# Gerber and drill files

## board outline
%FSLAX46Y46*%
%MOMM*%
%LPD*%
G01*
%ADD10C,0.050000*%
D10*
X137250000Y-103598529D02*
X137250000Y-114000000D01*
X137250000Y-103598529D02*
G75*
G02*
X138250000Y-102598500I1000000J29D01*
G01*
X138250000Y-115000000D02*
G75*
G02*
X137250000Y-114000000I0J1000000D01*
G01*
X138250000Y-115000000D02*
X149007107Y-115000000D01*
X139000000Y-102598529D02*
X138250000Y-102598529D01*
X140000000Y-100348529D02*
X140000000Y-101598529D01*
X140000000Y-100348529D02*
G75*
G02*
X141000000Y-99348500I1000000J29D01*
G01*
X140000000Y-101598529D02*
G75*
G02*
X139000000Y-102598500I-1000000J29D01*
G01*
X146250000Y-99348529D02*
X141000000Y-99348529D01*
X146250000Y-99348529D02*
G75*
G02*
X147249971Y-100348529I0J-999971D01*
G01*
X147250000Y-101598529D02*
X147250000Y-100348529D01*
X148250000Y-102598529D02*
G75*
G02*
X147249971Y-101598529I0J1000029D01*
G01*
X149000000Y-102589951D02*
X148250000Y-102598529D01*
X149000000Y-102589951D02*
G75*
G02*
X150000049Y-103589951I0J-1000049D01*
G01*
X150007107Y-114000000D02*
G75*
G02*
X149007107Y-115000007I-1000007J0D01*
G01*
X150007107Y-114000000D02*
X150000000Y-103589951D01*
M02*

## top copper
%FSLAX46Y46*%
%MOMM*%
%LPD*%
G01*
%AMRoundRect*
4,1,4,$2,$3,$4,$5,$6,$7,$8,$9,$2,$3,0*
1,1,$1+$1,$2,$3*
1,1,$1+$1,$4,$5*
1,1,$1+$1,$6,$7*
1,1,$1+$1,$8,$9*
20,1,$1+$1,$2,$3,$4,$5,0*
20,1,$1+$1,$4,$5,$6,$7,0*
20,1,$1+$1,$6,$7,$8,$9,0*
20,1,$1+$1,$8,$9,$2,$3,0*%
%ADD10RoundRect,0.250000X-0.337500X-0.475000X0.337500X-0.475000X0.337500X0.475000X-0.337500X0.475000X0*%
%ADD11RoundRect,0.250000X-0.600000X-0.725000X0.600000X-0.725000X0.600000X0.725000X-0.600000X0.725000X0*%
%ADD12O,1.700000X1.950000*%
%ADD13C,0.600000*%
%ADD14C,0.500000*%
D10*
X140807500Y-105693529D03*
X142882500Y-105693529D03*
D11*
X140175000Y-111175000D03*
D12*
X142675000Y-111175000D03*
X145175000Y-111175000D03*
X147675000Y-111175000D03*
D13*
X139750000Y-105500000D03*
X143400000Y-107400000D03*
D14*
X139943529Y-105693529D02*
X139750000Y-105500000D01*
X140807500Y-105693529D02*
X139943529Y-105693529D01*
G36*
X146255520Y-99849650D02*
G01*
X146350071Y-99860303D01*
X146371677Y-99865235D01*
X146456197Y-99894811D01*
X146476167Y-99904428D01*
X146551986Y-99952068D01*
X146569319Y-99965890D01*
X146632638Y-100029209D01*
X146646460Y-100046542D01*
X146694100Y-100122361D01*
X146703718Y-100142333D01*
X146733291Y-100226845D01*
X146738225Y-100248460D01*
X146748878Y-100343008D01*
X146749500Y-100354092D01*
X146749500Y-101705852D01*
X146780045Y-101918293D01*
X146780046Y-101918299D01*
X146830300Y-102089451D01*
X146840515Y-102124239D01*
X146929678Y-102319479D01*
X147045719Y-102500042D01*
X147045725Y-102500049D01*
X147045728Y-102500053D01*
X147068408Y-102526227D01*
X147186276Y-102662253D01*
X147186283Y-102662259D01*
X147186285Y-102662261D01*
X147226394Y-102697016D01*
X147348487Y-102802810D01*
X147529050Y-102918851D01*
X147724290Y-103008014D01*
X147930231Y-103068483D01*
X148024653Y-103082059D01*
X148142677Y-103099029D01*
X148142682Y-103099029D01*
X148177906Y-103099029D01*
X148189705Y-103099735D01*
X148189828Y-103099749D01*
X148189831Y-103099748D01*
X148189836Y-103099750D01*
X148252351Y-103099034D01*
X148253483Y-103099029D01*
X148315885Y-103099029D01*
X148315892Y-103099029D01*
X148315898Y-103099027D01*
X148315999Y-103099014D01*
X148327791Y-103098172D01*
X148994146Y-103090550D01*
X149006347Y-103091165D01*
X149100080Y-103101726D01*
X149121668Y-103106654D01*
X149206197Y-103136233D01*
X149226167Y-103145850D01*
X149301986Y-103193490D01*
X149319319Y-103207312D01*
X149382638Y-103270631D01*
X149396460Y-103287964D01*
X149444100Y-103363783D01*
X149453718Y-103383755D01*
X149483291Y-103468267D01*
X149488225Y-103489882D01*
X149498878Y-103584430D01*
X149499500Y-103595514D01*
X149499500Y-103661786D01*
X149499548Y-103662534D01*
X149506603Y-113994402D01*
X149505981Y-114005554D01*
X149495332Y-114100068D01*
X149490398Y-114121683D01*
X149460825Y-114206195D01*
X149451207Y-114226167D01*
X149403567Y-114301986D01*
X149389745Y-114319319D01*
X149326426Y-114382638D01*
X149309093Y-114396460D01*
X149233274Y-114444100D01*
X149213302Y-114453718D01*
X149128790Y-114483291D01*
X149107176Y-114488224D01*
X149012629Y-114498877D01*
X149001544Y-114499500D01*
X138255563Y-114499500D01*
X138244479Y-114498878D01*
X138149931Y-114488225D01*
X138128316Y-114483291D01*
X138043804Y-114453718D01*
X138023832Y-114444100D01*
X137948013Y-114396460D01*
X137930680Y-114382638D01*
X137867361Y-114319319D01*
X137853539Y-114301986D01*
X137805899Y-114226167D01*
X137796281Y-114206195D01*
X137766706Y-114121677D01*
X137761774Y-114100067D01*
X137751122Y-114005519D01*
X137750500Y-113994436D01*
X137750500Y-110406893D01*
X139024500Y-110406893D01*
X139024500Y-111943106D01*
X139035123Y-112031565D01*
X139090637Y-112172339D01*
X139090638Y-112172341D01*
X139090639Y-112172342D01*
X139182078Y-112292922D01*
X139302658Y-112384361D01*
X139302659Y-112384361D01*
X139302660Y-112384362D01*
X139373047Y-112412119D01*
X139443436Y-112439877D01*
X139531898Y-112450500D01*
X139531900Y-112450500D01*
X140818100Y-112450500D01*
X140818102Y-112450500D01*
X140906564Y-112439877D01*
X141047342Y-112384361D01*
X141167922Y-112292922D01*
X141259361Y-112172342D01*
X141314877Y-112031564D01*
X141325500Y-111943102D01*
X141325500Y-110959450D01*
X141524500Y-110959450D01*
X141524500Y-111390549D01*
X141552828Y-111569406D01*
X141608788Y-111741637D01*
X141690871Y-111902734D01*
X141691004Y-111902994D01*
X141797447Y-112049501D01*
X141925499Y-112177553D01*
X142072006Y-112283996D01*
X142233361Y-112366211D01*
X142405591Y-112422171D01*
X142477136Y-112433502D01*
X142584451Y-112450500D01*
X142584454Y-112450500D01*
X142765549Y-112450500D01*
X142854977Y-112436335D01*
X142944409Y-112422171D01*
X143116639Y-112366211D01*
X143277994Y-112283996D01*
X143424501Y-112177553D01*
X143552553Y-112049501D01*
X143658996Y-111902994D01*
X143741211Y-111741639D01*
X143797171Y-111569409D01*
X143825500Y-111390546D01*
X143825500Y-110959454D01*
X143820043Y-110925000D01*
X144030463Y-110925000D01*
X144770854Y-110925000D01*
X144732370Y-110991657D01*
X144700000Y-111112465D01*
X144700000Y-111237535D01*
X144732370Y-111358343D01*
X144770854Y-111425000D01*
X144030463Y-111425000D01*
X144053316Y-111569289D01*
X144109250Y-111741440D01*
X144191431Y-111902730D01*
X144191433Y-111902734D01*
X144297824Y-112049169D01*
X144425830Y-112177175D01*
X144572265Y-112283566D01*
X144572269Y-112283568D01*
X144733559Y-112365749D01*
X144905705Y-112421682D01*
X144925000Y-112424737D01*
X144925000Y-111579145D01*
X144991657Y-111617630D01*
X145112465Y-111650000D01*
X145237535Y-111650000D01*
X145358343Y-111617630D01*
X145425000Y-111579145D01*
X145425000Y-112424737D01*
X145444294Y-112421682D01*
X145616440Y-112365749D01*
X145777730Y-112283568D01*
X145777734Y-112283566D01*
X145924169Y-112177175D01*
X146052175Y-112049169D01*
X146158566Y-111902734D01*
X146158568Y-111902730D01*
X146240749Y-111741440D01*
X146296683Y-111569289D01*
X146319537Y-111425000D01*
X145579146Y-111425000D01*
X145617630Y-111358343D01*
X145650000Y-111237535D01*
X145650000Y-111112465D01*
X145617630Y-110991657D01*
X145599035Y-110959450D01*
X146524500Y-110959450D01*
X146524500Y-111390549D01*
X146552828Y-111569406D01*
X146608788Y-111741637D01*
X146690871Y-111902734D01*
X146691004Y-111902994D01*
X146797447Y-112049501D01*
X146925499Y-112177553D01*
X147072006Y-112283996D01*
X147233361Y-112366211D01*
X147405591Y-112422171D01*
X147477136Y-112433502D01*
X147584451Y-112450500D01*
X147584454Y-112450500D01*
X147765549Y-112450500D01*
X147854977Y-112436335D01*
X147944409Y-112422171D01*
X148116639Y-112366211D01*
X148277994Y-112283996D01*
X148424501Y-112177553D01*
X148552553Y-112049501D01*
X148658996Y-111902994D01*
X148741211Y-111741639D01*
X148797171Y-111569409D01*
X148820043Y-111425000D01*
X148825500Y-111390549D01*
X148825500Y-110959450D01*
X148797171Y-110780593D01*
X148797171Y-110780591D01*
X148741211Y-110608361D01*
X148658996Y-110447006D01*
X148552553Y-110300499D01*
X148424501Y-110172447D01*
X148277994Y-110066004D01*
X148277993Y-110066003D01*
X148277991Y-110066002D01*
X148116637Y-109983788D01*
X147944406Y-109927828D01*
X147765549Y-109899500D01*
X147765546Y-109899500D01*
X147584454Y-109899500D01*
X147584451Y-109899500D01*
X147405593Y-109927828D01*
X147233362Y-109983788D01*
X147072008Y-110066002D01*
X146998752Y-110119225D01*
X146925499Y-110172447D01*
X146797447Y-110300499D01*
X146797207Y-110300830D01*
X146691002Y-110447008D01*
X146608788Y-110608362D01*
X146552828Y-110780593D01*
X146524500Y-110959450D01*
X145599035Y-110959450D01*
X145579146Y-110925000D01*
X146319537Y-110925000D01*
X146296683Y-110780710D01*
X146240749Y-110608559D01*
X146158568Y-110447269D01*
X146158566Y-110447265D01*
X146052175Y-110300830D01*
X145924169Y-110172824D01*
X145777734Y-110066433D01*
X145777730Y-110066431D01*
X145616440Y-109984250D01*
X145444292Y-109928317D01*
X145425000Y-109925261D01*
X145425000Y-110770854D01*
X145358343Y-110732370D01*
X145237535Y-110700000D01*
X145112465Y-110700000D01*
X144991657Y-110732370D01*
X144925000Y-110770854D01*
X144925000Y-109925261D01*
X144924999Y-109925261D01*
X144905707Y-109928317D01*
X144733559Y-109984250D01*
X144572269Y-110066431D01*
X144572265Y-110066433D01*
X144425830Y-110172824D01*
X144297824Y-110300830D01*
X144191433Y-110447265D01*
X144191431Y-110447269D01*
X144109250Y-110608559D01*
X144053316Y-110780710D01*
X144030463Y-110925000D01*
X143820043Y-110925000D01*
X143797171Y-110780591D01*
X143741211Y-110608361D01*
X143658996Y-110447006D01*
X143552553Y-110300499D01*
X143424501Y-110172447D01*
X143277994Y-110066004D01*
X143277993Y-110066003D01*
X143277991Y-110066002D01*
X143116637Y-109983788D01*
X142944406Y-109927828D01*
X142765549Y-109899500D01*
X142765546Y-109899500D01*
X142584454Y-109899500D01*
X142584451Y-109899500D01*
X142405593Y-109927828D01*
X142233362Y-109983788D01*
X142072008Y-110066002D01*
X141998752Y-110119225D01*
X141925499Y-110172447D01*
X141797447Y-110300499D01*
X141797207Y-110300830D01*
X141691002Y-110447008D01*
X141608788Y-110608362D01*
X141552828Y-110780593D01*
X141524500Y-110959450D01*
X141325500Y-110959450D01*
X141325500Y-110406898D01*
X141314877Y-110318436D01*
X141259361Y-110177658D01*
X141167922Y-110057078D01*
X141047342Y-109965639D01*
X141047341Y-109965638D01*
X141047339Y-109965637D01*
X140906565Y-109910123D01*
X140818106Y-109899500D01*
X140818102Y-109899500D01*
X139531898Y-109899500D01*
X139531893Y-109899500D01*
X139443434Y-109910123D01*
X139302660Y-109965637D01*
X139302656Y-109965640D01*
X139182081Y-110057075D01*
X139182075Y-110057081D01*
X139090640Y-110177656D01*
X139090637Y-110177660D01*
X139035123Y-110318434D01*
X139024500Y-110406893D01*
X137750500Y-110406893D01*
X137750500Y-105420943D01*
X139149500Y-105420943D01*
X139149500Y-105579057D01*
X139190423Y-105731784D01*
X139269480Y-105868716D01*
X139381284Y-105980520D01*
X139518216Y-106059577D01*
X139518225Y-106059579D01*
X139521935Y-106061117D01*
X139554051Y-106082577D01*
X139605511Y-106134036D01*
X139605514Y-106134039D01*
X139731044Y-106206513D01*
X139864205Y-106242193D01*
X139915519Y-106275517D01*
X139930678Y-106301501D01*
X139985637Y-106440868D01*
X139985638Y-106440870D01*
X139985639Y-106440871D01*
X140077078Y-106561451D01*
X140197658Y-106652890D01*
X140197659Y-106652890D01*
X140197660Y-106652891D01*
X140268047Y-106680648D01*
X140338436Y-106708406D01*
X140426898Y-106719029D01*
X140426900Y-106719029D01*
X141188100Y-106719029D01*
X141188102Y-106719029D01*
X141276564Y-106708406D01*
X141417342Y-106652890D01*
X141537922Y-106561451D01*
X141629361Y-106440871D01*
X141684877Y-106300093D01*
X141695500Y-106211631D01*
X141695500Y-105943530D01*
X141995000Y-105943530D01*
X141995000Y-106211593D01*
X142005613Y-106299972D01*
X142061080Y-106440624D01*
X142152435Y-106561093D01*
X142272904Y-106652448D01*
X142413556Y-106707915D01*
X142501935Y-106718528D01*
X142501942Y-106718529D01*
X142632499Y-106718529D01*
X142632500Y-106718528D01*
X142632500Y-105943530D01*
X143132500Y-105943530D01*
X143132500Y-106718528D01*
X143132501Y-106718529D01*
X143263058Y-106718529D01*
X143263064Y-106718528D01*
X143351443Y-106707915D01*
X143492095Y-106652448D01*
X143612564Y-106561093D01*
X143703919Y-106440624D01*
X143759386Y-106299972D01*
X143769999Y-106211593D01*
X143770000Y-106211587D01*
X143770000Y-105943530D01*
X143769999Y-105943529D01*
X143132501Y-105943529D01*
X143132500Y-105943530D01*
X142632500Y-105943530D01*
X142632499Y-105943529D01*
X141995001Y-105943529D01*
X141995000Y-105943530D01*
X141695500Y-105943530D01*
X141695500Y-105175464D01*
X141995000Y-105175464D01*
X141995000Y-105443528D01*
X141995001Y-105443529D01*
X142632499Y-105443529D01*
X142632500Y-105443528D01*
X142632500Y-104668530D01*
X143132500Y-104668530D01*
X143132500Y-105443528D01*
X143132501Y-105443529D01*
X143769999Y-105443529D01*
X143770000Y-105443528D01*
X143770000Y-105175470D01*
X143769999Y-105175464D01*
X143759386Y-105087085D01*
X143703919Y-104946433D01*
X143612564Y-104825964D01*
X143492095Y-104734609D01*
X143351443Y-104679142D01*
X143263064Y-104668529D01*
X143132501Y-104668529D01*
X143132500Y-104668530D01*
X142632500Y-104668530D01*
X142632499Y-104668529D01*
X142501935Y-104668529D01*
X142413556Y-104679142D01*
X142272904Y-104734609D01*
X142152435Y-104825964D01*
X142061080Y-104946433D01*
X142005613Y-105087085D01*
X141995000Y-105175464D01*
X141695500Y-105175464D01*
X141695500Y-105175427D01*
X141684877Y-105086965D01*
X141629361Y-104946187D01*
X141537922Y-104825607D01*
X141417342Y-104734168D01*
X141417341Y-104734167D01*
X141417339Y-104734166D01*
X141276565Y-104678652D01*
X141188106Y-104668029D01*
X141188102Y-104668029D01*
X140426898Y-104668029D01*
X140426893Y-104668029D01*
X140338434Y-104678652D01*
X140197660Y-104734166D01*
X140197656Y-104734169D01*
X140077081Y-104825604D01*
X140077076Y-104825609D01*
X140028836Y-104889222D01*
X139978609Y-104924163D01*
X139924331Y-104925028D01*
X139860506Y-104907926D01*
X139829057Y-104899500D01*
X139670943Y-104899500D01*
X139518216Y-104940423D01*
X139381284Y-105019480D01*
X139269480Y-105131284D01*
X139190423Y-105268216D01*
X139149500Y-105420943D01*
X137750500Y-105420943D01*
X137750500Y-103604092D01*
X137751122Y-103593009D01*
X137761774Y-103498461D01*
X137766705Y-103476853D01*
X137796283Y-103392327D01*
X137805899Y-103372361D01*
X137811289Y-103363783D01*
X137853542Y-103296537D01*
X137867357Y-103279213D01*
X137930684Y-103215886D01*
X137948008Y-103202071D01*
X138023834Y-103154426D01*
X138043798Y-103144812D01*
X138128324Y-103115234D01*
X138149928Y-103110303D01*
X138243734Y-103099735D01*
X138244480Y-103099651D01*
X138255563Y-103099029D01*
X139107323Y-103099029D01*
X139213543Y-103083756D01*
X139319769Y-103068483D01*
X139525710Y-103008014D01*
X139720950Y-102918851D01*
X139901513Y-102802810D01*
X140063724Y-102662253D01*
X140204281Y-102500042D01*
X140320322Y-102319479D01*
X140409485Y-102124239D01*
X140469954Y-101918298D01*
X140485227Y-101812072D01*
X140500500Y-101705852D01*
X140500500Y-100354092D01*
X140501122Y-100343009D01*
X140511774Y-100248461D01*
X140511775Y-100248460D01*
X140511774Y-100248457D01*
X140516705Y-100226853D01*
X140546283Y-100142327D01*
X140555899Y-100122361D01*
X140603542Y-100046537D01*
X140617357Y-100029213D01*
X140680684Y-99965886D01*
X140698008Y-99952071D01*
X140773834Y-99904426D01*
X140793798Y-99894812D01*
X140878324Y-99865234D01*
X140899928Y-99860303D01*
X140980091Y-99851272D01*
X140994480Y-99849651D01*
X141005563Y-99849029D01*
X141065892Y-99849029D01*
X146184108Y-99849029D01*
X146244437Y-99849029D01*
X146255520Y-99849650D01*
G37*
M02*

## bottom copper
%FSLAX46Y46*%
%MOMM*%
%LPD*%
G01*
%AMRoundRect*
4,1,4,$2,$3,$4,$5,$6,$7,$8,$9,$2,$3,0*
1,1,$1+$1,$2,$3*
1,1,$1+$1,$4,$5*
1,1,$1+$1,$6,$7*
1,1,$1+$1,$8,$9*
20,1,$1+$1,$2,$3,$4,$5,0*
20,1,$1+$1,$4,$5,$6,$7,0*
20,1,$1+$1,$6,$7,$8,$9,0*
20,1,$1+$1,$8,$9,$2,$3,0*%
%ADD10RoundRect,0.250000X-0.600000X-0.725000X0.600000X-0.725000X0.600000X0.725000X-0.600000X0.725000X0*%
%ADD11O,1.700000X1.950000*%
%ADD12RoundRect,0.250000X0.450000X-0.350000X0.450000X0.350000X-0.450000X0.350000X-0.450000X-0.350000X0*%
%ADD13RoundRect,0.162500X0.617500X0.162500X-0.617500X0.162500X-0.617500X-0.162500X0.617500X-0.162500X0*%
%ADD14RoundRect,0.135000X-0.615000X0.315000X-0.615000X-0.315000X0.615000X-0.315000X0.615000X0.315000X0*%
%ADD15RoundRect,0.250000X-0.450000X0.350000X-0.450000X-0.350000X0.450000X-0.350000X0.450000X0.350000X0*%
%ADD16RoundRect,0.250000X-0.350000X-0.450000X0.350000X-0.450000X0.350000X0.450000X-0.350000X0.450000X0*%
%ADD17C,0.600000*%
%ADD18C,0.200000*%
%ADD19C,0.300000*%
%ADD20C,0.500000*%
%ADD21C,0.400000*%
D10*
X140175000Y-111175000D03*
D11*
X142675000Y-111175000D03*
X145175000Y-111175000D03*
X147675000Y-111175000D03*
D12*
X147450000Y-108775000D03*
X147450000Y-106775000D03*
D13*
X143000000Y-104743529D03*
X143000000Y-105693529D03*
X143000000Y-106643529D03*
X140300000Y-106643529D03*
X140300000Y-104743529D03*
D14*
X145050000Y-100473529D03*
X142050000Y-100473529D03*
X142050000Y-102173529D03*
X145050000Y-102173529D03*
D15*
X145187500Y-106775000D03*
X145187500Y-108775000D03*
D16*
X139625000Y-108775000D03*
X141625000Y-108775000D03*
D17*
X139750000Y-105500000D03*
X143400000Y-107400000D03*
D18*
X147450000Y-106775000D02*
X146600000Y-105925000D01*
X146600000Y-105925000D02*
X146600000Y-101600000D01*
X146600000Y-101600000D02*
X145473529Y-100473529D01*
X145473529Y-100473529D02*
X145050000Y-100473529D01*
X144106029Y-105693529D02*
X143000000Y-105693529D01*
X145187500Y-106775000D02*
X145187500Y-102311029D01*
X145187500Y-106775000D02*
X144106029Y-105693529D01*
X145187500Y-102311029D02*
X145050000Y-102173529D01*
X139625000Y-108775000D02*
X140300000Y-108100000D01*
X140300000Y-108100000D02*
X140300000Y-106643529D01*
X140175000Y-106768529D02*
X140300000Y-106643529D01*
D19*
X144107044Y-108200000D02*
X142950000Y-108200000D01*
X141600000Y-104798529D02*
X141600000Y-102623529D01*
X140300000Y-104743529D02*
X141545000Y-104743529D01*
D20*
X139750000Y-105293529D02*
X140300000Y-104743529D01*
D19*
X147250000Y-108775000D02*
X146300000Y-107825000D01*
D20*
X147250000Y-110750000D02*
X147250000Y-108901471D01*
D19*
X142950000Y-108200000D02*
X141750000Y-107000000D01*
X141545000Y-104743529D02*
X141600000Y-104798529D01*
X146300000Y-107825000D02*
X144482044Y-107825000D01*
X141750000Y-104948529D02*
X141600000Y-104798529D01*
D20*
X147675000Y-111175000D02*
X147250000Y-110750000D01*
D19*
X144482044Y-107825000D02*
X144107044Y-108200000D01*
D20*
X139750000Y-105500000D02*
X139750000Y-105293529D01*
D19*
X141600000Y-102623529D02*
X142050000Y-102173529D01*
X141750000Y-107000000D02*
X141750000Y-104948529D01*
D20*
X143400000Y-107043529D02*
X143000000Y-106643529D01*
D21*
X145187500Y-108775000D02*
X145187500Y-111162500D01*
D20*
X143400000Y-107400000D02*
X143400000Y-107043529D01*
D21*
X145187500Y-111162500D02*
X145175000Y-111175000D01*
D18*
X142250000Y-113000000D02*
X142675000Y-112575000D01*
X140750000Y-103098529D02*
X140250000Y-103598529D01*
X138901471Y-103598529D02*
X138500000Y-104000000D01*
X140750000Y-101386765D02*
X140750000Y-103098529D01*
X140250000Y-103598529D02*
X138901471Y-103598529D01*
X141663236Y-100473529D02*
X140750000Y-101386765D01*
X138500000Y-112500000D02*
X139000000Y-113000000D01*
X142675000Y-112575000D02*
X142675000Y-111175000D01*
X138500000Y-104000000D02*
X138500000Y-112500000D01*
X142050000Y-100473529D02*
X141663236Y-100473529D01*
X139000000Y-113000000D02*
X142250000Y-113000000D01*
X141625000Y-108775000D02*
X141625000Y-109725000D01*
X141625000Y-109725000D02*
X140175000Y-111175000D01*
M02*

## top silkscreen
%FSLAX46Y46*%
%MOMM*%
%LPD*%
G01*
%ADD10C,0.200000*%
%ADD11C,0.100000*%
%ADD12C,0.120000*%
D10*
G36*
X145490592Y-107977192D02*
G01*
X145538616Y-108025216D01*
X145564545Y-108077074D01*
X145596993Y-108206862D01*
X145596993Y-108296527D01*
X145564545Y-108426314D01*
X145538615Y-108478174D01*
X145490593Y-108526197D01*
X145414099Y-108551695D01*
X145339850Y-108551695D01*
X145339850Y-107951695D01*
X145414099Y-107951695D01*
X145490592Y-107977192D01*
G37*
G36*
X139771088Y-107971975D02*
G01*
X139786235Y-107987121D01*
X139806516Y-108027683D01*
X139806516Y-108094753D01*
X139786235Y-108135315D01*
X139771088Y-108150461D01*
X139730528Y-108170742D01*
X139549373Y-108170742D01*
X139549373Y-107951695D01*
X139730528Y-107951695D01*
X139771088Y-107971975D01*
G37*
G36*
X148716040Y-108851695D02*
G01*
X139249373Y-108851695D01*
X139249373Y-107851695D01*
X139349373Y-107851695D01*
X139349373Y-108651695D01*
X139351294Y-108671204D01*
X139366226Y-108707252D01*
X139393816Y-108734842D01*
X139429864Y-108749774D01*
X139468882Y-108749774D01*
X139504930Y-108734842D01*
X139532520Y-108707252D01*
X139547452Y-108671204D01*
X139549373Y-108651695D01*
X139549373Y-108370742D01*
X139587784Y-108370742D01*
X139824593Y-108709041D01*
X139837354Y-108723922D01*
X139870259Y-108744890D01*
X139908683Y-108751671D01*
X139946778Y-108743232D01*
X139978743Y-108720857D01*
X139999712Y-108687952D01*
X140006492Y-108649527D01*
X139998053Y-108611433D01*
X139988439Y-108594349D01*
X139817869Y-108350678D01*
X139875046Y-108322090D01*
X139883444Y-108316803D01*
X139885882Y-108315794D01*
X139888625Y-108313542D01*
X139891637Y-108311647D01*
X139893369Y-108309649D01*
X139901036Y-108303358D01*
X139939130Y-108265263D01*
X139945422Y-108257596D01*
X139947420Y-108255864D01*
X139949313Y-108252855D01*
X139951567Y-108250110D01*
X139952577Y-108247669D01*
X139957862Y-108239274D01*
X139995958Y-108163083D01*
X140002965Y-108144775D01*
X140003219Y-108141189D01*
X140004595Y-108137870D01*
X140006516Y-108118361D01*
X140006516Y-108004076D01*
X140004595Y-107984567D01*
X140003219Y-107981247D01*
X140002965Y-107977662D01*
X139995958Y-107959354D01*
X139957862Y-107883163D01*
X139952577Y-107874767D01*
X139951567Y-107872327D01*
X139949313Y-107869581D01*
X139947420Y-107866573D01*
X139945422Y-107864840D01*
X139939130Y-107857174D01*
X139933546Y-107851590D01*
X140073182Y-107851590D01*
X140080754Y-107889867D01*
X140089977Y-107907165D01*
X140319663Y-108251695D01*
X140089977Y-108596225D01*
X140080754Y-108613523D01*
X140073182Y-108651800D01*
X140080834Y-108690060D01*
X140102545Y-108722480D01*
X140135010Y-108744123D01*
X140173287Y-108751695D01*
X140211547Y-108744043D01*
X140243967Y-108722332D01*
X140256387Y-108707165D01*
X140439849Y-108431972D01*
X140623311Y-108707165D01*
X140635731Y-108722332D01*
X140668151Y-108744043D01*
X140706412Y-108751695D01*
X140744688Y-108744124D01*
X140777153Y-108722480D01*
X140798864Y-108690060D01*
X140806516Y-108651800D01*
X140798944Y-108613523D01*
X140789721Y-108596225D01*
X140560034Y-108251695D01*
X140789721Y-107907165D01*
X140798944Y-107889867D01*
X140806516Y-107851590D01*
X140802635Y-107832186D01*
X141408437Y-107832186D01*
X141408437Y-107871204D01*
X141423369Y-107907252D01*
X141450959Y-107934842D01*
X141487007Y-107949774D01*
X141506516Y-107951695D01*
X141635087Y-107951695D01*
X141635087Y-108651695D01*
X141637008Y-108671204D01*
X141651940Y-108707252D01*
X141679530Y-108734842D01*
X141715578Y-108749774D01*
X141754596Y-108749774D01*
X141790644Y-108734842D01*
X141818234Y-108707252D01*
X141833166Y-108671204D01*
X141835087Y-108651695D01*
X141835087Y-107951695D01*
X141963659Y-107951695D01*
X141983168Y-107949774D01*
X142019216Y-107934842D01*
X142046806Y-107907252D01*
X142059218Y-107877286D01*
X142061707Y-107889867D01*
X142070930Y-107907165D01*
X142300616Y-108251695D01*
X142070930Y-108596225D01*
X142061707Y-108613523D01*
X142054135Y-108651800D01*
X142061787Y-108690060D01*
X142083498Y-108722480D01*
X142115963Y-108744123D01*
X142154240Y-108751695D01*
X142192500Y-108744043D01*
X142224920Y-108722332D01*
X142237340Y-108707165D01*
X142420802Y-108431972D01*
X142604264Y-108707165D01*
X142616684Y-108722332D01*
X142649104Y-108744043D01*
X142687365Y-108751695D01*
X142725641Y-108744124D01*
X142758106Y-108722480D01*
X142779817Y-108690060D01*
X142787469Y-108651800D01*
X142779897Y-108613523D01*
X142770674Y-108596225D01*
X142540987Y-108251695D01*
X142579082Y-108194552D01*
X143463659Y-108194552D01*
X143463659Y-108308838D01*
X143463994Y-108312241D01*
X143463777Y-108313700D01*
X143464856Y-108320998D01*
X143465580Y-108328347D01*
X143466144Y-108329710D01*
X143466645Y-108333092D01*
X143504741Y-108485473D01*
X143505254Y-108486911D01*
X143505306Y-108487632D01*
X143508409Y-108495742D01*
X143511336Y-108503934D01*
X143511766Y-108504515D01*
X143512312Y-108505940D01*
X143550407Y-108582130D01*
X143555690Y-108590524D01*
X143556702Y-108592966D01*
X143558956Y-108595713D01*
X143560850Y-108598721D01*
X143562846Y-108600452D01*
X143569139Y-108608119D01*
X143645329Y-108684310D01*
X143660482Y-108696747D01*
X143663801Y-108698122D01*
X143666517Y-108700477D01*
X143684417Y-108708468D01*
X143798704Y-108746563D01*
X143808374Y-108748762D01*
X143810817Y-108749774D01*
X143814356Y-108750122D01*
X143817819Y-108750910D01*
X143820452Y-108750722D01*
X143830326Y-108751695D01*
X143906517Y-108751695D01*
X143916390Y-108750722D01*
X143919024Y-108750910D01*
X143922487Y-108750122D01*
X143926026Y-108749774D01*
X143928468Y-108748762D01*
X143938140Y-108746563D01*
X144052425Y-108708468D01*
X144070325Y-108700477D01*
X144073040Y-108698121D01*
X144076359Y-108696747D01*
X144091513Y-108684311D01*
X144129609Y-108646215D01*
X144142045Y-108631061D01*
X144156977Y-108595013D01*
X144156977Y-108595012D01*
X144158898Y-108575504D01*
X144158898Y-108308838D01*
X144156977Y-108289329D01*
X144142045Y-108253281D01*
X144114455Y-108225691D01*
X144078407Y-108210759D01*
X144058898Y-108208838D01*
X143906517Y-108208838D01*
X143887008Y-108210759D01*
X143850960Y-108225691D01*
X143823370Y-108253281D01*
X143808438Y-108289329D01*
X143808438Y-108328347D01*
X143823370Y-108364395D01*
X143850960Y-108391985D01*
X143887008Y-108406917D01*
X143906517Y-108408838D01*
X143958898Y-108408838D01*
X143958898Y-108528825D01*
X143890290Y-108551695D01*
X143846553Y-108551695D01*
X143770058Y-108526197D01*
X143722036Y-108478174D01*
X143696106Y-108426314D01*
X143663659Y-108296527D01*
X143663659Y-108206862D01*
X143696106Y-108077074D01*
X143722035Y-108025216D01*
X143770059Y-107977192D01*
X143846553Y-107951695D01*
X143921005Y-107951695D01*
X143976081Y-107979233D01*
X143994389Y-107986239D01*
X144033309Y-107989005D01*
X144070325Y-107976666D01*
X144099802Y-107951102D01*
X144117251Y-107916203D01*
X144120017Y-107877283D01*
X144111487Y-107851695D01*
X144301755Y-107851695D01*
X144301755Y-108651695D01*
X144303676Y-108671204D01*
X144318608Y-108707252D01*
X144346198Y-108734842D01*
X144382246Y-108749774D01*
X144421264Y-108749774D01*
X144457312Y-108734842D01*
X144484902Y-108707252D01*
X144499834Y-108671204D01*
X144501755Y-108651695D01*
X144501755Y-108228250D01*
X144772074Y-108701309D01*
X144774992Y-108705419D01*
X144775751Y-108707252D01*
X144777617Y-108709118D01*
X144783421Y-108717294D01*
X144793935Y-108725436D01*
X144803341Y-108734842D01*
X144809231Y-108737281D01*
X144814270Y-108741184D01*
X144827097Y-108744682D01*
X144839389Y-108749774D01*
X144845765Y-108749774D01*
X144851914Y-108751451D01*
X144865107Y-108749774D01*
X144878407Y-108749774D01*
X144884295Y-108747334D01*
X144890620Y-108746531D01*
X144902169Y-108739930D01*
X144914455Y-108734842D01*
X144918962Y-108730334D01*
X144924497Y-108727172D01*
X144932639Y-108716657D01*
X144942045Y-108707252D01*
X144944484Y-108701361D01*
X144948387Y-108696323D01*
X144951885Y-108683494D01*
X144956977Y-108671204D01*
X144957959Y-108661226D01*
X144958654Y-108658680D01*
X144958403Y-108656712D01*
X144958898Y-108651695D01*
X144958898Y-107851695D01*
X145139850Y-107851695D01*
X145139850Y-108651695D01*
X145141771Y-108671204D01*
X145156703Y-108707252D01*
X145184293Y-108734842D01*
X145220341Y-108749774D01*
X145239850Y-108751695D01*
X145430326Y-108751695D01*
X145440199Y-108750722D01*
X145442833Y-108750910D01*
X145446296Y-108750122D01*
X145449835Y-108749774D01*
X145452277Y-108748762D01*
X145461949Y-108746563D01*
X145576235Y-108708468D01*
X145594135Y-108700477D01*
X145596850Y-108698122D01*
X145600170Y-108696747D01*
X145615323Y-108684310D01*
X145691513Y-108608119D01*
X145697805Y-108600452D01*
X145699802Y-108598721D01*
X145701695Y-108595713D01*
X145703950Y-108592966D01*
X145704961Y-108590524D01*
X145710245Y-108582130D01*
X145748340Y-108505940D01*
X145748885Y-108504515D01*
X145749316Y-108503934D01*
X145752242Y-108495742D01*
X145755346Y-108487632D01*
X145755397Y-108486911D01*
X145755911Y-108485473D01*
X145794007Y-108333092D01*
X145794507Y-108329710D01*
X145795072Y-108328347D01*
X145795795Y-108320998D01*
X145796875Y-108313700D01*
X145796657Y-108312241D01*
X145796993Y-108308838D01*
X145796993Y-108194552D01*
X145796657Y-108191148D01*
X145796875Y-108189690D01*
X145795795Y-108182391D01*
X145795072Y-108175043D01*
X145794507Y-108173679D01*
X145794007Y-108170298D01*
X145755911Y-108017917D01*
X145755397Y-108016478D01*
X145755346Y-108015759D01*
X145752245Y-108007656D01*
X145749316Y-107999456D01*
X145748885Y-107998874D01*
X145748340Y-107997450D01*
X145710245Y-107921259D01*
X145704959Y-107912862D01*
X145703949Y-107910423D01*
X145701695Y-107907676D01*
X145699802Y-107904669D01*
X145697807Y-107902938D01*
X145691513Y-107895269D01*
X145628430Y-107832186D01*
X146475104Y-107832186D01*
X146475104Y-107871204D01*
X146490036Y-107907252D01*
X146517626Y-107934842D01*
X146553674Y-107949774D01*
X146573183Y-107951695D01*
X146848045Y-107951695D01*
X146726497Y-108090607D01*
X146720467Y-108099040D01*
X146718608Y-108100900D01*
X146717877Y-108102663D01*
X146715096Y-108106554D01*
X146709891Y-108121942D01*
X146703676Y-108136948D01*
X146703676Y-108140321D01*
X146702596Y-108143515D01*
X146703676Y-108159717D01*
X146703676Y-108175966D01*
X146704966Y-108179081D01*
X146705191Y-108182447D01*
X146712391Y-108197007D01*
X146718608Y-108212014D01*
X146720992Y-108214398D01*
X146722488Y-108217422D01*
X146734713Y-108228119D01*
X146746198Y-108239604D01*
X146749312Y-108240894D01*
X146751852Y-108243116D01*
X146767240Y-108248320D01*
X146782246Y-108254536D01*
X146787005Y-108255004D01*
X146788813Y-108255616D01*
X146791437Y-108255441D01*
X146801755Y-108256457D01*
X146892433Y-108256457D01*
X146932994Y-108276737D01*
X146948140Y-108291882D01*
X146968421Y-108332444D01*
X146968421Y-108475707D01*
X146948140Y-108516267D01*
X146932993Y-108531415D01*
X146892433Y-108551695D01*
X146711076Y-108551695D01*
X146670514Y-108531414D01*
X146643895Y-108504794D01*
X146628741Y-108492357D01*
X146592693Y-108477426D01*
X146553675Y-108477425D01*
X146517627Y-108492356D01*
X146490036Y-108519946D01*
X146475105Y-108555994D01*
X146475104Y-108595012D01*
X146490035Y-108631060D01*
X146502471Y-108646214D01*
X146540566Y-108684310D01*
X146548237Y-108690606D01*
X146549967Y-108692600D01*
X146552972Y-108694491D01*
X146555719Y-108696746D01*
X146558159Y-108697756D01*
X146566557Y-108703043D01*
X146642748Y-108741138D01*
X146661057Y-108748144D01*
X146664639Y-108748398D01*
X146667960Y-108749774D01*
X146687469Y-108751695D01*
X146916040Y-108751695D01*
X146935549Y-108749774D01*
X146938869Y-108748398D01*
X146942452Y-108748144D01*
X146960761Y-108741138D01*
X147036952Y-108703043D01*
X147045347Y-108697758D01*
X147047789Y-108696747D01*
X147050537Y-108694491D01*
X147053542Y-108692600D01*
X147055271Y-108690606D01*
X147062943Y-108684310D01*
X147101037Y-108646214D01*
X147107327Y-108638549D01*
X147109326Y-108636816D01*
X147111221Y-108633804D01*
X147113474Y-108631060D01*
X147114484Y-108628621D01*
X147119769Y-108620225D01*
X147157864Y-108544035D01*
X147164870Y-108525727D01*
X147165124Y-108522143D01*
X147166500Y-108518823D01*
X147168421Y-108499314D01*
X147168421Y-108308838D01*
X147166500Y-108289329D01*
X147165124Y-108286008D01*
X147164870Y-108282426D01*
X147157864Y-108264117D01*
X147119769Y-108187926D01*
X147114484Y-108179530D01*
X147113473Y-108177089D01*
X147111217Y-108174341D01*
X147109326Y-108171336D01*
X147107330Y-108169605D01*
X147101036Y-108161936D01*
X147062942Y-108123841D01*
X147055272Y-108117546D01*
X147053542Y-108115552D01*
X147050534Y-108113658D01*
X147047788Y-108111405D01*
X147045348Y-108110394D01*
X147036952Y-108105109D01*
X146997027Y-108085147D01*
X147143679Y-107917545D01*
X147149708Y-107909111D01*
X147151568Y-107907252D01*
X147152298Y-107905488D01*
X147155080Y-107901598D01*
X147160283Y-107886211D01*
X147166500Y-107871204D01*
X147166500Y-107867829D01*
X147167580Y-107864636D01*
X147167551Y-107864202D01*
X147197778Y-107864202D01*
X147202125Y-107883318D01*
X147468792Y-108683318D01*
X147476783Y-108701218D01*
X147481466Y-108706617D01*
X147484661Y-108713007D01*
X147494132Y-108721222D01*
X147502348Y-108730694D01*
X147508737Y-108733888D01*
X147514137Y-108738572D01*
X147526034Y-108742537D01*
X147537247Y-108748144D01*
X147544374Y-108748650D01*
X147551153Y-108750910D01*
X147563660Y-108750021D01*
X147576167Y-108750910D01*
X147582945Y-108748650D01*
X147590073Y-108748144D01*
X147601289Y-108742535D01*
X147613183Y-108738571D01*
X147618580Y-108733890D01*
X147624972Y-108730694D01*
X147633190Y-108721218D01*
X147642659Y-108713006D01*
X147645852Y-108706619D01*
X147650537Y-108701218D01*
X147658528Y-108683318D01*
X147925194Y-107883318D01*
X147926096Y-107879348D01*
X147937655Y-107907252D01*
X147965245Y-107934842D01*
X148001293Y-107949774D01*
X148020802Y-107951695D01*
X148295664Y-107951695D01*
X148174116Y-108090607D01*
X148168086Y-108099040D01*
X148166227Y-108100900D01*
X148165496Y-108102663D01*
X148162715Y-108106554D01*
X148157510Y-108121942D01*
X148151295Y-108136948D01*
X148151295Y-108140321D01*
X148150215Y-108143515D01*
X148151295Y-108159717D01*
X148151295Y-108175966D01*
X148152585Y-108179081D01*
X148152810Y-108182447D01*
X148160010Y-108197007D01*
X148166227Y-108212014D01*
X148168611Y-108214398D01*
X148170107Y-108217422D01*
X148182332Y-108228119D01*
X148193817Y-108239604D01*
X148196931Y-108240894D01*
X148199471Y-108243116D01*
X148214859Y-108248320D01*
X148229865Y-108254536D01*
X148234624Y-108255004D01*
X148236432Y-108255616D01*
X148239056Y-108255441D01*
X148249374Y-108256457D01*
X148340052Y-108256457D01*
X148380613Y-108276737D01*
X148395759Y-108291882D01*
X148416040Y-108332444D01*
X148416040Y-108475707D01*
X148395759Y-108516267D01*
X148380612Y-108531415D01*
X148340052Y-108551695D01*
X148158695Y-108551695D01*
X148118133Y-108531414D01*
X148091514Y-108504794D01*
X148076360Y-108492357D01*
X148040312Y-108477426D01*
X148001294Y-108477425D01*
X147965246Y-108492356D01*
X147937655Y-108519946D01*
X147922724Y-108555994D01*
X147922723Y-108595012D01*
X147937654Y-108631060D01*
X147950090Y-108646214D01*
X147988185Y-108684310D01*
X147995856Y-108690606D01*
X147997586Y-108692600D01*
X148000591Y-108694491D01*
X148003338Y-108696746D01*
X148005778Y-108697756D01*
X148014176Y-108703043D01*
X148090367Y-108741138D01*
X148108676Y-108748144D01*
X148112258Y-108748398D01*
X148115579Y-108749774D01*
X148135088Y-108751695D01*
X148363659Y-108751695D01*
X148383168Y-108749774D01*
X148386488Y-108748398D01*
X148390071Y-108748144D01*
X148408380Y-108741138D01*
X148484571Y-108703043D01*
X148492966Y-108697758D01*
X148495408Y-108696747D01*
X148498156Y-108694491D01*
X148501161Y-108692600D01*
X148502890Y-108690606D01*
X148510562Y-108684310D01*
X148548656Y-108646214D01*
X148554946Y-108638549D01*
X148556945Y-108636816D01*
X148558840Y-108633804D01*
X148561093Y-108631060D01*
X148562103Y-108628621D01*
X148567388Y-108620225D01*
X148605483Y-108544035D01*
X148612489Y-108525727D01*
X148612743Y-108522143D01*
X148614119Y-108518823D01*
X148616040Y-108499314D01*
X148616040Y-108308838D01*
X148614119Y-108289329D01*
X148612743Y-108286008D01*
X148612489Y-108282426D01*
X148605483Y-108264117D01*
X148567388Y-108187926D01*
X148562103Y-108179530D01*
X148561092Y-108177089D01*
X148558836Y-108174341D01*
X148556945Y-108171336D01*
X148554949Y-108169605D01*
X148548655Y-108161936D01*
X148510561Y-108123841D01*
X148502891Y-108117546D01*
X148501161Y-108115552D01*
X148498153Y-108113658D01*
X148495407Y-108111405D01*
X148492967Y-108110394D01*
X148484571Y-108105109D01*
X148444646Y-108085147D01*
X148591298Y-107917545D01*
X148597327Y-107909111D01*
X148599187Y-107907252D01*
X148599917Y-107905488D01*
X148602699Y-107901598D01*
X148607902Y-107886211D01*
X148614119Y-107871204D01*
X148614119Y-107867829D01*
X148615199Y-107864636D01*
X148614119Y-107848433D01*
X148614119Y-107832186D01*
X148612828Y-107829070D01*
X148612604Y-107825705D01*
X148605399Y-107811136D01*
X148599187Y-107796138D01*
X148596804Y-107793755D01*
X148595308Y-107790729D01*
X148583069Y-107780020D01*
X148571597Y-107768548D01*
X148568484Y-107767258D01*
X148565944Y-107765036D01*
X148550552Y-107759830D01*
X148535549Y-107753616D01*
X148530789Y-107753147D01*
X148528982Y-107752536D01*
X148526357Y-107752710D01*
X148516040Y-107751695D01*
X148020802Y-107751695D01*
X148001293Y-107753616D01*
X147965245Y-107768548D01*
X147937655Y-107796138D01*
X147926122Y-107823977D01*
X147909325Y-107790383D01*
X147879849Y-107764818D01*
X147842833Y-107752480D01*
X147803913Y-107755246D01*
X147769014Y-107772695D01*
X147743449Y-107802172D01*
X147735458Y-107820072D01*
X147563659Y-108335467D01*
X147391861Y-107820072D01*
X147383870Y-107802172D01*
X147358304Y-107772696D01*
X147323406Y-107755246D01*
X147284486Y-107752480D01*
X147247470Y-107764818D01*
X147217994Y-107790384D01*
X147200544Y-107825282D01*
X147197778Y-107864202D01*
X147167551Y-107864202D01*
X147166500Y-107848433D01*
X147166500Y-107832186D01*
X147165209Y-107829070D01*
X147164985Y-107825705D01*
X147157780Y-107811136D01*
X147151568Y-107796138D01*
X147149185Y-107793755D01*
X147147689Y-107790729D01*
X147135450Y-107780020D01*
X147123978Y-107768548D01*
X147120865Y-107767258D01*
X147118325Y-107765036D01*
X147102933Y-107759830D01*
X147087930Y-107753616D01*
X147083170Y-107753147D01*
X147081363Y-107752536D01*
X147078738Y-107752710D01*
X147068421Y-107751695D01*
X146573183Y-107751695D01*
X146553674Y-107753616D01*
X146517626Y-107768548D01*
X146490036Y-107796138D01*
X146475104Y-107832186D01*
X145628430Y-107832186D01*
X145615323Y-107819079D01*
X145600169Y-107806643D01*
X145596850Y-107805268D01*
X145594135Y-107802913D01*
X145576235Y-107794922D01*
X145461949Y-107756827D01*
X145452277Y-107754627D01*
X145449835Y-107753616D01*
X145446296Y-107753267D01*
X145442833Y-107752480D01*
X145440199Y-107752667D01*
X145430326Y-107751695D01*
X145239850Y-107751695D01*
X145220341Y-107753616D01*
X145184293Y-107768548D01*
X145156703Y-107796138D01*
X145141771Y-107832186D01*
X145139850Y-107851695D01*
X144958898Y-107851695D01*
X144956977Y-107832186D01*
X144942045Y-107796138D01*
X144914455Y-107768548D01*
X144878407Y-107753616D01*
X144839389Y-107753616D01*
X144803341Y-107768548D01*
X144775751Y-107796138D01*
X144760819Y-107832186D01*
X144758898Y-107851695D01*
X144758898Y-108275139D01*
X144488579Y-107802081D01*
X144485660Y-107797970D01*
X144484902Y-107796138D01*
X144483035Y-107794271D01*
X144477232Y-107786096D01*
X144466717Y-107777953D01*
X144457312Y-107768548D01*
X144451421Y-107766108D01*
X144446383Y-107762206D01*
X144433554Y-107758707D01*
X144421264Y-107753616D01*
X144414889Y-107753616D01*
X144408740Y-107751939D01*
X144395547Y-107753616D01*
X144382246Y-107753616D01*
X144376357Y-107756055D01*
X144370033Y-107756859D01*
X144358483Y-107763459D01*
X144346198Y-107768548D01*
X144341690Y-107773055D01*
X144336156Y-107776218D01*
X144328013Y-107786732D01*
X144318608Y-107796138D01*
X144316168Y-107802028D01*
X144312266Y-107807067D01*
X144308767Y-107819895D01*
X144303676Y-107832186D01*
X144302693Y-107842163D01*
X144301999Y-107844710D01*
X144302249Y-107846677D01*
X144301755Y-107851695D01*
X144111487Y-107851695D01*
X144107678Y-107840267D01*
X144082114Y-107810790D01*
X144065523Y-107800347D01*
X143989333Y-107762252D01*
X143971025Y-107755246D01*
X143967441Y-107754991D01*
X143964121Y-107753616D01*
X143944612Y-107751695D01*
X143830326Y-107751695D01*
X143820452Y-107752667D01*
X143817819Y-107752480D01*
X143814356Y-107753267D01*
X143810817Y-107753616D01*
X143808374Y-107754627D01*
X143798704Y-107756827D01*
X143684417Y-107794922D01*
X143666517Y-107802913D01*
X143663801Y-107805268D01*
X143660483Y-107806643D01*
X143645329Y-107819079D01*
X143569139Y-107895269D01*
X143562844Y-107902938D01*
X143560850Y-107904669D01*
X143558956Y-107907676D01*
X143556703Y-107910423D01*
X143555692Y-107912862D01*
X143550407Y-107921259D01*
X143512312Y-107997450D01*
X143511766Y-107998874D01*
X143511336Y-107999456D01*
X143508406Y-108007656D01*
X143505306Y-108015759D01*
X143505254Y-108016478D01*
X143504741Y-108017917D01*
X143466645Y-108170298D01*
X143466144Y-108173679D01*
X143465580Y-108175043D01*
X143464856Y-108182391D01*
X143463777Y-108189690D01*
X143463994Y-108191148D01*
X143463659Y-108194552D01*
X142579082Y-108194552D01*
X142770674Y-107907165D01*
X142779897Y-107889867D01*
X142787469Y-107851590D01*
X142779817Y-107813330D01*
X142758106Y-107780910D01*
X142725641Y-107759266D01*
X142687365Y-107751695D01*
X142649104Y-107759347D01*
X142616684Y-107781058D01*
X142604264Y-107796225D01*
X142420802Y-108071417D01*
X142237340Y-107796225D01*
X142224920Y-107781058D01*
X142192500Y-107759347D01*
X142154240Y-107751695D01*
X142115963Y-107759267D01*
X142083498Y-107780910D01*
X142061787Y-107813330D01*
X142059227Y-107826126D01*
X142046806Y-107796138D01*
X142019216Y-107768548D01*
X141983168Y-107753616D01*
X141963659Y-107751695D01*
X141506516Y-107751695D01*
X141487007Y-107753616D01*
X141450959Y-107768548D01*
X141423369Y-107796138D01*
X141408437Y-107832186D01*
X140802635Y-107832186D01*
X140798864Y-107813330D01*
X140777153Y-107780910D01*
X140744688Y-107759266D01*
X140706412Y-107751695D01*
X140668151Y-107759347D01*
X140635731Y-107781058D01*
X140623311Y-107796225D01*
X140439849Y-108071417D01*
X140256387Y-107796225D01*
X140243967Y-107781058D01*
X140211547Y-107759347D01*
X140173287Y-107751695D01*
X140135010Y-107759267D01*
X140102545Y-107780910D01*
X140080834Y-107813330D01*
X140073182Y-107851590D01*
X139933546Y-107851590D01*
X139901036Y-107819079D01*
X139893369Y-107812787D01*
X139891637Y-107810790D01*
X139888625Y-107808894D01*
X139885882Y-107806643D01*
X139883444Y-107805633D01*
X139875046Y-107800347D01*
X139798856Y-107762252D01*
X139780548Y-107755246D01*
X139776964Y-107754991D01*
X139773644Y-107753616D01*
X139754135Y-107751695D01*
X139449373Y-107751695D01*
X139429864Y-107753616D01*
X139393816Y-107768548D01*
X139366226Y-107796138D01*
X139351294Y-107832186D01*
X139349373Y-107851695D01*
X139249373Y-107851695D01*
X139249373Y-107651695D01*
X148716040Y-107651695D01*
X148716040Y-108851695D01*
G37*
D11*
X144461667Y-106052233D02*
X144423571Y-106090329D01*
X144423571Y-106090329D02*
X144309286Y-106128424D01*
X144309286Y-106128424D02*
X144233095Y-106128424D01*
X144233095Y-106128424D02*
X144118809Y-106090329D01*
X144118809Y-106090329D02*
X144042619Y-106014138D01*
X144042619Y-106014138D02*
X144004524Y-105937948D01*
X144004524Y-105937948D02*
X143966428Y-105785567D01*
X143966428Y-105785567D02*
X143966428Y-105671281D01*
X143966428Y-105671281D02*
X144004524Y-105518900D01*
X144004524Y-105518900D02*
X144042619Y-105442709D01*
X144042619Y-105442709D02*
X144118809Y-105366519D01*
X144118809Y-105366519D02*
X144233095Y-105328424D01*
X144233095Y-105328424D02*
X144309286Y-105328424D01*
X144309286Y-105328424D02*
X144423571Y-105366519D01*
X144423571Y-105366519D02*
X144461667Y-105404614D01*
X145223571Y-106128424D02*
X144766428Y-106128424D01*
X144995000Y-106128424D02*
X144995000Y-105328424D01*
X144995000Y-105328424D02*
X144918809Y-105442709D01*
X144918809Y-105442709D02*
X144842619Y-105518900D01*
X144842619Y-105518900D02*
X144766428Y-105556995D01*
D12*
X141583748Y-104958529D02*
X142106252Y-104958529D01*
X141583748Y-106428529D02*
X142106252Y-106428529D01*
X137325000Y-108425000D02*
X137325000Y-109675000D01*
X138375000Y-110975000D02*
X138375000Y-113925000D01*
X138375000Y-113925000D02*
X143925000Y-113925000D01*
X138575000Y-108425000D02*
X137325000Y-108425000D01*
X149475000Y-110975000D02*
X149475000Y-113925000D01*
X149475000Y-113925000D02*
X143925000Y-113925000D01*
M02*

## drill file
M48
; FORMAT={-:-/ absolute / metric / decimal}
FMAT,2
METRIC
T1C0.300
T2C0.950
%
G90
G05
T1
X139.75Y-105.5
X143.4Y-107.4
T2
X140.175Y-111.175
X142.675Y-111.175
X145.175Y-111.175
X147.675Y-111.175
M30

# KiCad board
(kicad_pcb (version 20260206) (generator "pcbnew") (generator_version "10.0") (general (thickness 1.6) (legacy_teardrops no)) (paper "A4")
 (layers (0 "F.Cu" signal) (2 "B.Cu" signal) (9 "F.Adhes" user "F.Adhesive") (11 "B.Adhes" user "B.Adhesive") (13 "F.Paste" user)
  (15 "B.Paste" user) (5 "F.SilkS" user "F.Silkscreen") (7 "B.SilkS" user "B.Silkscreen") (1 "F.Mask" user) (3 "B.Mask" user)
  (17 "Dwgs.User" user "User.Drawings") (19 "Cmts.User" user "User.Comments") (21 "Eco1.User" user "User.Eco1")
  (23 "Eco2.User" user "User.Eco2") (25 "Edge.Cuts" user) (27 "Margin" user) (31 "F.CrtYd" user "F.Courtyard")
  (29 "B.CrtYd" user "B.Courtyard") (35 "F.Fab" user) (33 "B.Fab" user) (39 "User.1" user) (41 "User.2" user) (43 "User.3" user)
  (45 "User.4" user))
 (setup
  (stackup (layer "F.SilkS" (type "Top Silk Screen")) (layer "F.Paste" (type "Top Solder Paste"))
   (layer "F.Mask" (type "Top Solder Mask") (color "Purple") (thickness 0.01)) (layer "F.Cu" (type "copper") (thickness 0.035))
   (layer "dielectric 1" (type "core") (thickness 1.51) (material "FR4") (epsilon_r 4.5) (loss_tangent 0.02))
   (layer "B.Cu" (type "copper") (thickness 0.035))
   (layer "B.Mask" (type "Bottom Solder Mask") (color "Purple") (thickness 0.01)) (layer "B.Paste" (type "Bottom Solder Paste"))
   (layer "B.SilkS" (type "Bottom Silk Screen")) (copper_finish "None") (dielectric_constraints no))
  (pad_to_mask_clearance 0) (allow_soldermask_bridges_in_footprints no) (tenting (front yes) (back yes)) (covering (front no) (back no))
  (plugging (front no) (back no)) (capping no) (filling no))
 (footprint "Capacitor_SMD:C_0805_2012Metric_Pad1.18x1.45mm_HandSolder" (layer "F.Cu") (at 141.845 105.693529)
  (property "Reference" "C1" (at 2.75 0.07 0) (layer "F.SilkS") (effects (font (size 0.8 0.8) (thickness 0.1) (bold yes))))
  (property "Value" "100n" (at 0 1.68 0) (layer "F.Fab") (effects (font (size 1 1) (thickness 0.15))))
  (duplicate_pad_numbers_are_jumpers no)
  (fp_line (start -0.261252 -0.735) (end 0.261252 -0.735) (stroke (width 0.12) (type solid)) (layer "F.SilkS"))
  (fp_line (start -0.261252 0.735) (end 0.261252 0.735) (stroke (width 0.12) (type solid)) (layer "F.SilkS"))
  (pad "1" smd roundrect (at -1.0375 0) (size 1.175 1.45) (layers "F.Cu" "F.Mask" "F.Paste") (roundrect_rratio 0.212766) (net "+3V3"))
  (pad "2" smd roundrect (at 1.0375 0) (size 1.175 1.45) (layers "F.Cu" "F.Mask" "F.Paste") (roundrect_rratio 0.212766) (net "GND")))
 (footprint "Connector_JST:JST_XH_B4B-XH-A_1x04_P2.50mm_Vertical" (layer "F.Cu") (at 140.175 111.175)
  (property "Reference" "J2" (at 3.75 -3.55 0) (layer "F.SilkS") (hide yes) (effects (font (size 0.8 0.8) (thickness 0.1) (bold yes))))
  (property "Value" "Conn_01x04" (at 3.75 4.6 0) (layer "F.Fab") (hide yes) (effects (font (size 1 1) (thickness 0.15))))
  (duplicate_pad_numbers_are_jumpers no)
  (fp_line (start -2.85 -2.75) (end -2.85 -1.5) (stroke (width 0.12) (type solid)) (layer "F.SilkS"))
  (fp_line (start -1.8 -0.2) (end -1.8 2.75) (stroke (width 0.12) (type solid)) (layer "F.SilkS"))
  (fp_line (start -1.8 2.75) (end 3.75 2.75) (stroke (width 0.12) (type solid)) (layer "F.SilkS"))
  (fp_line (start -1.6 -2.75) (end -2.85 -2.75) (stroke (width 0.12) (type solid)) (layer "F.SilkS"))
  (fp_line (start 9.3 -0.2) (end 9.3 2.75) (stroke (width 0.12) (type solid)) (layer "F.SilkS"))
  (fp_line (start 9.3 2.75) (end 3.75 2.75) (stroke (width 0.12) (type solid)) (layer "F.SilkS"))
  (pad "1" thru_hole roundrect (at 0 0) (size 1.7 1.95) (drill 0.95) (layers "*.Cu" "*.Mask") (remove_unused_layers no)
   (roundrect_rratio 0.147059) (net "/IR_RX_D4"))
  (pad "2" thru_hole oval (at 2.5 0) (size 1.7 1.95) (drill 0.95) (layers "*.Cu" "*.Mask") (remove_unused_layers no) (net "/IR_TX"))
  (pad "3" thru_hole oval (at 5 0) (size 1.7 1.95) (drill 0.95) (layers "*.Cu" "*.Mask") (remove_unused_layers no) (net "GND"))
  (pad "4" thru_hole oval (at 7.5 0) (size 1.7 1.95) (drill 0.95) (layers "*.Cu" "*.Mask") (remove_unused_layers no) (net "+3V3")))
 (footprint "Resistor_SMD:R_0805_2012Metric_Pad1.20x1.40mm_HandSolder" (layer "B.Cu") (at 147.45 107.775 90)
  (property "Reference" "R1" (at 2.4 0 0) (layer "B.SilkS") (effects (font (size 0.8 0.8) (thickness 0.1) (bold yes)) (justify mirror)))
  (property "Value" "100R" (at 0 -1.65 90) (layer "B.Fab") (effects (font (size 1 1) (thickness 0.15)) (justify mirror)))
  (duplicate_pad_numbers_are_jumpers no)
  (pad "1" smd roundrect (at -1 0 90) (size 1.2 1.4) (layers "B.Cu" "B.Mask" "B.Paste") (roundrect_rratio 0.208333) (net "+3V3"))
  (pad "2" smd roundrect (at 1 0 90) (size 1.2 1.4) (layers "B.Cu" "B.Mask" "B.Paste") (roundrect_rratio 0.208333) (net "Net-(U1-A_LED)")))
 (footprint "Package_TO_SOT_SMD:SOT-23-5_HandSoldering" (layer "B.Cu") (at 141.65 105.693529 180)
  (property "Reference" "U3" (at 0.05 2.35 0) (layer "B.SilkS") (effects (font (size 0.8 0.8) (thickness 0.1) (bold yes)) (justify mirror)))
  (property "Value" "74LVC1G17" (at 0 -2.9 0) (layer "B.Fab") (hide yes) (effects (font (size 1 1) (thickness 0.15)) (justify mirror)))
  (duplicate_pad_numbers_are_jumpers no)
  (pad "1" smd roundrect (at -1.35 0.95 180) (size 1.56 0.65) (layers "B.Cu" "B.Mask" "B.Paste") (roundrect_rratio 0.25)
   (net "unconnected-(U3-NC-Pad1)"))
  (pad "2" smd roundrect (at -1.35 0 180) (size 1.56 0.65) (layers "B.Cu" "B.Mask" "B.Paste") (roundrect_rratio 0.25) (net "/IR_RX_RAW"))
  (pad "3" smd roundrect (at -1.35 -0.95 180) (size 1.56 0.65) (layers "B.Cu" "B.Mask" "B.Paste") (roundrect_rratio 0.25) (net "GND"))
  (pad "4" smd roundrect (at 1.35 -0.95 180) (size 1.56 0.65) (layers "B.Cu" "B.Mask" "B.Paste") (roundrect_rratio 0.25)
   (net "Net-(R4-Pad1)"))
  (pad "5" smd roundrect (at 1.35 0.95 180) (size 1.56 0.65) (layers "B.Cu" "B.Mask" "B.Paste") (roundrect_rratio 0.25) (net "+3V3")))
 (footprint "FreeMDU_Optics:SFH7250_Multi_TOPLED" (layer "B.Cu") (at 143.55 101.323529 -90)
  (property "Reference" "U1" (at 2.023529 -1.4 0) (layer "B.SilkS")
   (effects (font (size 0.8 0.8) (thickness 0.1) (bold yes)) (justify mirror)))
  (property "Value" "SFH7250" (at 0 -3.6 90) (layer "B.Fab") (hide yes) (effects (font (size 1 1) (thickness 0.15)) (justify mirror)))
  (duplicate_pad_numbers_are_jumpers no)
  (pad "1" smd roundrect (at -0.85 -1.5 270) (size 0.9 1.5) (layers "B.Cu" "B.Mask" "B.Paste") (roundrect_rratio 0.15)
   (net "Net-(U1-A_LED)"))
  (pad "2" smd roundrect (at -0.85 1.5 270) (size 0.9 1.5) (layers "B.Cu" "B.Mask" "B.Paste") (roundrect_rratio 0.15) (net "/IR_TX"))
  (pad "3" smd roundrect (at 0.85 1.5 270) (size 0.9 1.5) (layers "B.Cu" "B.Mask" "B.Paste") (roundrect_rratio 0.15) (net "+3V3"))
  (pad "4" smd roundrect (at 0.85 -1.5 270) (size 0.9 1.5) (layers "B.Cu" "B.Mask" "B.Paste") (roundrect_rratio 0.15) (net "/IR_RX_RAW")))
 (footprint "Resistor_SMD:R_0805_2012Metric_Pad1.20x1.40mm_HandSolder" (layer "B.Cu") (at 145.1875 107.775 -90)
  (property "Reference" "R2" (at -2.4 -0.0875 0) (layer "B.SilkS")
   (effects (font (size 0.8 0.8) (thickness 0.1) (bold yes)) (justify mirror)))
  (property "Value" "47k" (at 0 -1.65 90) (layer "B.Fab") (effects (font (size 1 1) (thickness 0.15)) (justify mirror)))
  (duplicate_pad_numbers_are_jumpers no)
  (pad "1" smd roundrect (at -1 0 270) (size 1.2 1.4) (layers "B.Cu" "B.Mask" "B.Paste") (roundrect_rratio 0.208333) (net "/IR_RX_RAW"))
  (pad "2" smd roundrect (at 1 0 270) (size 1.2 1.4) (layers "B.Cu" "B.Mask" "B.Paste") (roundrect_rratio 0.208333) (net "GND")))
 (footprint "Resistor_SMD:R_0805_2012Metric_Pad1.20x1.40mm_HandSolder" (layer "B.Cu") (at 140.625 108.775)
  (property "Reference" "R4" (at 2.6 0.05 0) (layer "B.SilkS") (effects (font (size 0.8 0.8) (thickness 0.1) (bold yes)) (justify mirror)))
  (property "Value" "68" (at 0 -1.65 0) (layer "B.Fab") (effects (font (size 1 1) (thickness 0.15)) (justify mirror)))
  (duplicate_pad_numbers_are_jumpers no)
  (pad "1" smd roundrect (at -1 0) (size 1.2 1.4) (layers "B.Cu" "B.Mask" "B.Paste") (roundrect_rratio 0.208333) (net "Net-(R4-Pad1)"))
  (pad "2" smd roundrect (at 1 0) (size 1.2 1.4) (layers "B.Cu" "B.Mask" "B.Paste") (roundrect_rratio 0.208333) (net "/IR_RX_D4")))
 (gr_line (start 137.25 103.598529) (end 137.25 114) (stroke (width 0.05) (type default)) (layer "Edge.Cuts"))
 (gr_arc (start 137.25 103.598529) (mid 137.542893 102.891422) (end 138.25 102.598529) (stroke (width 0.05) (type default))
  (layer "Edge.Cuts"))
 (gr_arc (start 138.25 115) (mid 137.542893 114.707107) (end 137.25 114) (stroke (width 0.05) (type default)) (layer "Edge.Cuts"))
 (gr_line (start 138.25 115) (end 149.007107 115) (stroke (width 0.05) (type default)) (layer "Edge.Cuts"))
 (gr_line (start 139 102.598529) (end 138.25 102.598529) (stroke (width 0.05) (type default)) (layer "Edge.Cuts"))
 (gr_line (start 140 100.348529) (end 140 101.598529) (stroke (width 0.05) (type default)) (layer "Edge.Cuts"))
 (gr_arc (start 140 100.348529) (mid 140.292893 99.641422) (end 141 99.348529) (stroke (width 0.05) (type default)) (layer "Edge.Cuts"))
 (gr_arc (start 140 101.598529) (mid 139.707107 102.305636) (end 139 102.598529) (stroke (width 0.05) (type default)) (layer "Edge.Cuts"))
 (gr_line (start 146.25 99.348529) (end 141 99.348529) (stroke (width 0.05) (type default)) (layer "Edge.Cuts"))
 (gr_arc (start 146.25 99.348529) (mid 146.957107 99.641422) (end 147.25 100.348529) (stroke (width 0.05) (type default))
  (layer "Edge.Cuts"))
 (gr_line (start 147.25 101.598529) (end 147.25 100.348529) (stroke (width 0.05) (type default)) (layer "Edge.Cuts"))
 (gr_arc (start 148.25 102.598529) (mid 147.542893 102.305636) (end 147.25 101.598529) (stroke (width 0.05) (type default))
  (layer "Edge.Cuts"))
 (gr_line (start 149 102.589951) (end 148.25 102.598529) (stroke (width 0.05) (type default)) (layer "Edge.Cuts"))
 (gr_arc (start 149 102.589951) (mid 149.707107 102.882844) (end 150 103.589951) (stroke (width 0.05) (type default)) (layer "Edge.Cuts"))
 (gr_arc (start 150.007107 114) (mid 149.714214 114.707107) (end 149.007107 115) (stroke (width 0.05) (type default)) (layer "Edge.Cuts"))
 (gr_line (start 150.007107 114) (end 150 103.589951) (stroke (width 0.05) (type default)) (layer "Edge.Cuts"))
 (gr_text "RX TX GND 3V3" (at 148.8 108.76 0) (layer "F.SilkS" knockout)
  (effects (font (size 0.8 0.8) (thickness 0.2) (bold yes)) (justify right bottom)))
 (segment (start 147.45 106.775) (end 146.6 105.925) (width 0.2) (layer "B.Cu") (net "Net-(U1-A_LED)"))
 (segment (start 146.6 105.925) (end 146.6 101.6) (width 0.2) (layer "B.Cu") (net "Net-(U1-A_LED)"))
 (segment (start 146.6 101.6) (end 145.473529 100.473529) (width 0.2) (layer "B.Cu") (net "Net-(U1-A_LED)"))
 (segment (start 145.473529 100.473529) (end 145.05 100.473529) (width 0.2) (layer "B.Cu") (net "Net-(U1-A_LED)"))
 (segment (start 144.106029 105.693529) (end 143 105.693529) (width 0.2) (layer "B.Cu") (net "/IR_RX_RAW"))
 (segment (start 145.1875 106.775) (end 145.1875 102.311029) (width 0.2) (layer "B.Cu") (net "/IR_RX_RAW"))
 (segment (start 145.1875 106.775) (end 144.106029 105.693529) (width 0.2) (layer "B.Cu") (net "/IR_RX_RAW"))
 (segment (start 145.1875 102.311029) (end 145.05 102.173529) (width 0.2) (layer "B.Cu") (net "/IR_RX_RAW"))
 (segment (start 139.625 108.775) (end 140.3 108.1) (width 0.2) (layer "B.Cu") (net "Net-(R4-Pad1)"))
 (segment (start 140.3 108.1) (end 140.3 106.643529) (width 0.2) (layer "B.Cu") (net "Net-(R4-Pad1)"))
 (segment (start 140.175 106.768529) (end 140.3 106.643529) (width 0.2) (layer "B.Cu") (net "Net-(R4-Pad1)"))
 (segment (start 139.943529 105.693529) (end 139.75 105.5) (width 0.5) (layer "F.Cu") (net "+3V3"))
 (segment (start 140.8075 105.693529) (end 139.943529 105.693529) (width 0.5) (layer "F.Cu") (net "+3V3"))
 (via (at 139.75 105.5) (size 0.6) (drill 0.3) (layers "F.Cu" "B.Cu") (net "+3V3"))
 (segment (start 144.107044 108.2) (end 142.95 108.2) (width 0.3) (layer "B.Cu") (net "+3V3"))
 (segment (start 141.6 104.798529) (end 141.6 102.623529) (width 0.3) (layer "B.Cu") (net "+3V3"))
 (segment (start 140.3 104.743529) (end 141.545 104.743529) (width 0.3) (layer "B.Cu") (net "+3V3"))
 (segment (start 139.75 105.293529) (end 140.3 104.743529) (width 0.5) (layer "B.Cu") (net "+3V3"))
 (segment (start 147.25 108.775) (end 146.3 107.825) (width 0.3) (layer "B.Cu") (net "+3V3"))
 (segment (start 147.25 110.75) (end 147.25 108.901471) (width 0.5) (layer "B.Cu") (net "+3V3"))
 (segment (start 142.95 108.2) (end 141.75 107) (width 0.3) (layer "B.Cu") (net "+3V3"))
 (segment (start 141.545 104.743529) (end 141.6 104.798529) (width 0.3) (layer "B.Cu") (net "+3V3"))
 (segment (start 146.3 107.825) (end 144.482044 107.825) (width 0.3) (layer "B.Cu") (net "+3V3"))
 (segment (start 141.75 104.948529) (end 141.6 104.798529) (width 0.3) (layer "B.Cu") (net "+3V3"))
 (segment (start 147.675 111.175) (end 147.25 110.75) (width 0.5) (layer "B.Cu") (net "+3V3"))
 (segment (start 144.482044 107.825) (end 144.107044 108.2) (width 0.3) (layer "B.Cu") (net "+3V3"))
 (segment (start 139.75 105.5) (end 139.75 105.293529) (width 0.5) (layer "B.Cu") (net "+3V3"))
 (segment (start 141.6 102.623529) (end 142.05 102.173529) (width 0.3) (layer "B.Cu") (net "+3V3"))
 (segment (start 141.75 107) (end 141.75 104.948529) (width 0.3) (layer "B.Cu") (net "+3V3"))
 (via (at 143.4 107.4) (size 0.6) (drill 0.3) (layers "F.Cu" "B.Cu") (free yes) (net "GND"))
 (segment (start 143.4 107.043529) (end 143 106.643529) (width 0.5) (layer "B.Cu") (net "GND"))
 (segment (start 145.1875 108.775) (end 145.1875 111.1625) (width 0.4) (layer "B.Cu") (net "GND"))
 (segment (start 143.4 107.4) (end 143.4 107.043529) (width 0.5) (layer "B.Cu") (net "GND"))
 (segment (start 145.1875 111.1625) (end 145.175 111.175) (width 0.4) (layer "B.Cu") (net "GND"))
 (segment (start 142.25 113) (end 142.675 112.575) (width 0.2) (layer "B.Cu") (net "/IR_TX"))
 (segment (start 140.75 103.098529) (end 140.25 103.598529) (width 0.2) (layer "B.Cu") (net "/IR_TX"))
 (segment (start 138.901471 103.598529) (end 138.5 104) (width 0.2) (layer "B.Cu") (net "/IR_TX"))
 (segment (start 140.75 101.386765) (end 140.75 103.098529) (width 0.2) (layer "B.Cu") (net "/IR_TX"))
 (segment (start 140.25 103.598529) (end 138.901471 103.598529) (width 0.2) (layer "B.Cu") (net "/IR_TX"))
 (segment (start 141.663236 100.473529) (end 140.75 101.386765) (width 0.2) (layer "B.Cu") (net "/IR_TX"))
 (segment (start 138.5 112.5) (end 139 113) (width 0.2) (layer "B.Cu") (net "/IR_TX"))
 (segment (start 142.675 112.575) (end 142.675 111.175) (width 0.2) (layer "B.Cu") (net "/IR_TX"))
 (segment (start 138.5 104) (end 138.5 112.5) (width 0.2) (layer "B.Cu") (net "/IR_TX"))
 (segment (start 142.05 100.473529) (end 141.663236 100.473529) (width 0.2) (layer "B.Cu") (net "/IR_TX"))
 (segment (start 139 113) (end 142.25 113) (width 0.2) (layer "B.Cu") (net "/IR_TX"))
 (segment (start 141.625 108.775) (end 141.625 109.725) (width 0.2) (layer "B.Cu") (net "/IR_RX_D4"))
 (segment (start 141.625 109.725) (end 140.175 111.175) (width 0.2) (layer "B.Cu") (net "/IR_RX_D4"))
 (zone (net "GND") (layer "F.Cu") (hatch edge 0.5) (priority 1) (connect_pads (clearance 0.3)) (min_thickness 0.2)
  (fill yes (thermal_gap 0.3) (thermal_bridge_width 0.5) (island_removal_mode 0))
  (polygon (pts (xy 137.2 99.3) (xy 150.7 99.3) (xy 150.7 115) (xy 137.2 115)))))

